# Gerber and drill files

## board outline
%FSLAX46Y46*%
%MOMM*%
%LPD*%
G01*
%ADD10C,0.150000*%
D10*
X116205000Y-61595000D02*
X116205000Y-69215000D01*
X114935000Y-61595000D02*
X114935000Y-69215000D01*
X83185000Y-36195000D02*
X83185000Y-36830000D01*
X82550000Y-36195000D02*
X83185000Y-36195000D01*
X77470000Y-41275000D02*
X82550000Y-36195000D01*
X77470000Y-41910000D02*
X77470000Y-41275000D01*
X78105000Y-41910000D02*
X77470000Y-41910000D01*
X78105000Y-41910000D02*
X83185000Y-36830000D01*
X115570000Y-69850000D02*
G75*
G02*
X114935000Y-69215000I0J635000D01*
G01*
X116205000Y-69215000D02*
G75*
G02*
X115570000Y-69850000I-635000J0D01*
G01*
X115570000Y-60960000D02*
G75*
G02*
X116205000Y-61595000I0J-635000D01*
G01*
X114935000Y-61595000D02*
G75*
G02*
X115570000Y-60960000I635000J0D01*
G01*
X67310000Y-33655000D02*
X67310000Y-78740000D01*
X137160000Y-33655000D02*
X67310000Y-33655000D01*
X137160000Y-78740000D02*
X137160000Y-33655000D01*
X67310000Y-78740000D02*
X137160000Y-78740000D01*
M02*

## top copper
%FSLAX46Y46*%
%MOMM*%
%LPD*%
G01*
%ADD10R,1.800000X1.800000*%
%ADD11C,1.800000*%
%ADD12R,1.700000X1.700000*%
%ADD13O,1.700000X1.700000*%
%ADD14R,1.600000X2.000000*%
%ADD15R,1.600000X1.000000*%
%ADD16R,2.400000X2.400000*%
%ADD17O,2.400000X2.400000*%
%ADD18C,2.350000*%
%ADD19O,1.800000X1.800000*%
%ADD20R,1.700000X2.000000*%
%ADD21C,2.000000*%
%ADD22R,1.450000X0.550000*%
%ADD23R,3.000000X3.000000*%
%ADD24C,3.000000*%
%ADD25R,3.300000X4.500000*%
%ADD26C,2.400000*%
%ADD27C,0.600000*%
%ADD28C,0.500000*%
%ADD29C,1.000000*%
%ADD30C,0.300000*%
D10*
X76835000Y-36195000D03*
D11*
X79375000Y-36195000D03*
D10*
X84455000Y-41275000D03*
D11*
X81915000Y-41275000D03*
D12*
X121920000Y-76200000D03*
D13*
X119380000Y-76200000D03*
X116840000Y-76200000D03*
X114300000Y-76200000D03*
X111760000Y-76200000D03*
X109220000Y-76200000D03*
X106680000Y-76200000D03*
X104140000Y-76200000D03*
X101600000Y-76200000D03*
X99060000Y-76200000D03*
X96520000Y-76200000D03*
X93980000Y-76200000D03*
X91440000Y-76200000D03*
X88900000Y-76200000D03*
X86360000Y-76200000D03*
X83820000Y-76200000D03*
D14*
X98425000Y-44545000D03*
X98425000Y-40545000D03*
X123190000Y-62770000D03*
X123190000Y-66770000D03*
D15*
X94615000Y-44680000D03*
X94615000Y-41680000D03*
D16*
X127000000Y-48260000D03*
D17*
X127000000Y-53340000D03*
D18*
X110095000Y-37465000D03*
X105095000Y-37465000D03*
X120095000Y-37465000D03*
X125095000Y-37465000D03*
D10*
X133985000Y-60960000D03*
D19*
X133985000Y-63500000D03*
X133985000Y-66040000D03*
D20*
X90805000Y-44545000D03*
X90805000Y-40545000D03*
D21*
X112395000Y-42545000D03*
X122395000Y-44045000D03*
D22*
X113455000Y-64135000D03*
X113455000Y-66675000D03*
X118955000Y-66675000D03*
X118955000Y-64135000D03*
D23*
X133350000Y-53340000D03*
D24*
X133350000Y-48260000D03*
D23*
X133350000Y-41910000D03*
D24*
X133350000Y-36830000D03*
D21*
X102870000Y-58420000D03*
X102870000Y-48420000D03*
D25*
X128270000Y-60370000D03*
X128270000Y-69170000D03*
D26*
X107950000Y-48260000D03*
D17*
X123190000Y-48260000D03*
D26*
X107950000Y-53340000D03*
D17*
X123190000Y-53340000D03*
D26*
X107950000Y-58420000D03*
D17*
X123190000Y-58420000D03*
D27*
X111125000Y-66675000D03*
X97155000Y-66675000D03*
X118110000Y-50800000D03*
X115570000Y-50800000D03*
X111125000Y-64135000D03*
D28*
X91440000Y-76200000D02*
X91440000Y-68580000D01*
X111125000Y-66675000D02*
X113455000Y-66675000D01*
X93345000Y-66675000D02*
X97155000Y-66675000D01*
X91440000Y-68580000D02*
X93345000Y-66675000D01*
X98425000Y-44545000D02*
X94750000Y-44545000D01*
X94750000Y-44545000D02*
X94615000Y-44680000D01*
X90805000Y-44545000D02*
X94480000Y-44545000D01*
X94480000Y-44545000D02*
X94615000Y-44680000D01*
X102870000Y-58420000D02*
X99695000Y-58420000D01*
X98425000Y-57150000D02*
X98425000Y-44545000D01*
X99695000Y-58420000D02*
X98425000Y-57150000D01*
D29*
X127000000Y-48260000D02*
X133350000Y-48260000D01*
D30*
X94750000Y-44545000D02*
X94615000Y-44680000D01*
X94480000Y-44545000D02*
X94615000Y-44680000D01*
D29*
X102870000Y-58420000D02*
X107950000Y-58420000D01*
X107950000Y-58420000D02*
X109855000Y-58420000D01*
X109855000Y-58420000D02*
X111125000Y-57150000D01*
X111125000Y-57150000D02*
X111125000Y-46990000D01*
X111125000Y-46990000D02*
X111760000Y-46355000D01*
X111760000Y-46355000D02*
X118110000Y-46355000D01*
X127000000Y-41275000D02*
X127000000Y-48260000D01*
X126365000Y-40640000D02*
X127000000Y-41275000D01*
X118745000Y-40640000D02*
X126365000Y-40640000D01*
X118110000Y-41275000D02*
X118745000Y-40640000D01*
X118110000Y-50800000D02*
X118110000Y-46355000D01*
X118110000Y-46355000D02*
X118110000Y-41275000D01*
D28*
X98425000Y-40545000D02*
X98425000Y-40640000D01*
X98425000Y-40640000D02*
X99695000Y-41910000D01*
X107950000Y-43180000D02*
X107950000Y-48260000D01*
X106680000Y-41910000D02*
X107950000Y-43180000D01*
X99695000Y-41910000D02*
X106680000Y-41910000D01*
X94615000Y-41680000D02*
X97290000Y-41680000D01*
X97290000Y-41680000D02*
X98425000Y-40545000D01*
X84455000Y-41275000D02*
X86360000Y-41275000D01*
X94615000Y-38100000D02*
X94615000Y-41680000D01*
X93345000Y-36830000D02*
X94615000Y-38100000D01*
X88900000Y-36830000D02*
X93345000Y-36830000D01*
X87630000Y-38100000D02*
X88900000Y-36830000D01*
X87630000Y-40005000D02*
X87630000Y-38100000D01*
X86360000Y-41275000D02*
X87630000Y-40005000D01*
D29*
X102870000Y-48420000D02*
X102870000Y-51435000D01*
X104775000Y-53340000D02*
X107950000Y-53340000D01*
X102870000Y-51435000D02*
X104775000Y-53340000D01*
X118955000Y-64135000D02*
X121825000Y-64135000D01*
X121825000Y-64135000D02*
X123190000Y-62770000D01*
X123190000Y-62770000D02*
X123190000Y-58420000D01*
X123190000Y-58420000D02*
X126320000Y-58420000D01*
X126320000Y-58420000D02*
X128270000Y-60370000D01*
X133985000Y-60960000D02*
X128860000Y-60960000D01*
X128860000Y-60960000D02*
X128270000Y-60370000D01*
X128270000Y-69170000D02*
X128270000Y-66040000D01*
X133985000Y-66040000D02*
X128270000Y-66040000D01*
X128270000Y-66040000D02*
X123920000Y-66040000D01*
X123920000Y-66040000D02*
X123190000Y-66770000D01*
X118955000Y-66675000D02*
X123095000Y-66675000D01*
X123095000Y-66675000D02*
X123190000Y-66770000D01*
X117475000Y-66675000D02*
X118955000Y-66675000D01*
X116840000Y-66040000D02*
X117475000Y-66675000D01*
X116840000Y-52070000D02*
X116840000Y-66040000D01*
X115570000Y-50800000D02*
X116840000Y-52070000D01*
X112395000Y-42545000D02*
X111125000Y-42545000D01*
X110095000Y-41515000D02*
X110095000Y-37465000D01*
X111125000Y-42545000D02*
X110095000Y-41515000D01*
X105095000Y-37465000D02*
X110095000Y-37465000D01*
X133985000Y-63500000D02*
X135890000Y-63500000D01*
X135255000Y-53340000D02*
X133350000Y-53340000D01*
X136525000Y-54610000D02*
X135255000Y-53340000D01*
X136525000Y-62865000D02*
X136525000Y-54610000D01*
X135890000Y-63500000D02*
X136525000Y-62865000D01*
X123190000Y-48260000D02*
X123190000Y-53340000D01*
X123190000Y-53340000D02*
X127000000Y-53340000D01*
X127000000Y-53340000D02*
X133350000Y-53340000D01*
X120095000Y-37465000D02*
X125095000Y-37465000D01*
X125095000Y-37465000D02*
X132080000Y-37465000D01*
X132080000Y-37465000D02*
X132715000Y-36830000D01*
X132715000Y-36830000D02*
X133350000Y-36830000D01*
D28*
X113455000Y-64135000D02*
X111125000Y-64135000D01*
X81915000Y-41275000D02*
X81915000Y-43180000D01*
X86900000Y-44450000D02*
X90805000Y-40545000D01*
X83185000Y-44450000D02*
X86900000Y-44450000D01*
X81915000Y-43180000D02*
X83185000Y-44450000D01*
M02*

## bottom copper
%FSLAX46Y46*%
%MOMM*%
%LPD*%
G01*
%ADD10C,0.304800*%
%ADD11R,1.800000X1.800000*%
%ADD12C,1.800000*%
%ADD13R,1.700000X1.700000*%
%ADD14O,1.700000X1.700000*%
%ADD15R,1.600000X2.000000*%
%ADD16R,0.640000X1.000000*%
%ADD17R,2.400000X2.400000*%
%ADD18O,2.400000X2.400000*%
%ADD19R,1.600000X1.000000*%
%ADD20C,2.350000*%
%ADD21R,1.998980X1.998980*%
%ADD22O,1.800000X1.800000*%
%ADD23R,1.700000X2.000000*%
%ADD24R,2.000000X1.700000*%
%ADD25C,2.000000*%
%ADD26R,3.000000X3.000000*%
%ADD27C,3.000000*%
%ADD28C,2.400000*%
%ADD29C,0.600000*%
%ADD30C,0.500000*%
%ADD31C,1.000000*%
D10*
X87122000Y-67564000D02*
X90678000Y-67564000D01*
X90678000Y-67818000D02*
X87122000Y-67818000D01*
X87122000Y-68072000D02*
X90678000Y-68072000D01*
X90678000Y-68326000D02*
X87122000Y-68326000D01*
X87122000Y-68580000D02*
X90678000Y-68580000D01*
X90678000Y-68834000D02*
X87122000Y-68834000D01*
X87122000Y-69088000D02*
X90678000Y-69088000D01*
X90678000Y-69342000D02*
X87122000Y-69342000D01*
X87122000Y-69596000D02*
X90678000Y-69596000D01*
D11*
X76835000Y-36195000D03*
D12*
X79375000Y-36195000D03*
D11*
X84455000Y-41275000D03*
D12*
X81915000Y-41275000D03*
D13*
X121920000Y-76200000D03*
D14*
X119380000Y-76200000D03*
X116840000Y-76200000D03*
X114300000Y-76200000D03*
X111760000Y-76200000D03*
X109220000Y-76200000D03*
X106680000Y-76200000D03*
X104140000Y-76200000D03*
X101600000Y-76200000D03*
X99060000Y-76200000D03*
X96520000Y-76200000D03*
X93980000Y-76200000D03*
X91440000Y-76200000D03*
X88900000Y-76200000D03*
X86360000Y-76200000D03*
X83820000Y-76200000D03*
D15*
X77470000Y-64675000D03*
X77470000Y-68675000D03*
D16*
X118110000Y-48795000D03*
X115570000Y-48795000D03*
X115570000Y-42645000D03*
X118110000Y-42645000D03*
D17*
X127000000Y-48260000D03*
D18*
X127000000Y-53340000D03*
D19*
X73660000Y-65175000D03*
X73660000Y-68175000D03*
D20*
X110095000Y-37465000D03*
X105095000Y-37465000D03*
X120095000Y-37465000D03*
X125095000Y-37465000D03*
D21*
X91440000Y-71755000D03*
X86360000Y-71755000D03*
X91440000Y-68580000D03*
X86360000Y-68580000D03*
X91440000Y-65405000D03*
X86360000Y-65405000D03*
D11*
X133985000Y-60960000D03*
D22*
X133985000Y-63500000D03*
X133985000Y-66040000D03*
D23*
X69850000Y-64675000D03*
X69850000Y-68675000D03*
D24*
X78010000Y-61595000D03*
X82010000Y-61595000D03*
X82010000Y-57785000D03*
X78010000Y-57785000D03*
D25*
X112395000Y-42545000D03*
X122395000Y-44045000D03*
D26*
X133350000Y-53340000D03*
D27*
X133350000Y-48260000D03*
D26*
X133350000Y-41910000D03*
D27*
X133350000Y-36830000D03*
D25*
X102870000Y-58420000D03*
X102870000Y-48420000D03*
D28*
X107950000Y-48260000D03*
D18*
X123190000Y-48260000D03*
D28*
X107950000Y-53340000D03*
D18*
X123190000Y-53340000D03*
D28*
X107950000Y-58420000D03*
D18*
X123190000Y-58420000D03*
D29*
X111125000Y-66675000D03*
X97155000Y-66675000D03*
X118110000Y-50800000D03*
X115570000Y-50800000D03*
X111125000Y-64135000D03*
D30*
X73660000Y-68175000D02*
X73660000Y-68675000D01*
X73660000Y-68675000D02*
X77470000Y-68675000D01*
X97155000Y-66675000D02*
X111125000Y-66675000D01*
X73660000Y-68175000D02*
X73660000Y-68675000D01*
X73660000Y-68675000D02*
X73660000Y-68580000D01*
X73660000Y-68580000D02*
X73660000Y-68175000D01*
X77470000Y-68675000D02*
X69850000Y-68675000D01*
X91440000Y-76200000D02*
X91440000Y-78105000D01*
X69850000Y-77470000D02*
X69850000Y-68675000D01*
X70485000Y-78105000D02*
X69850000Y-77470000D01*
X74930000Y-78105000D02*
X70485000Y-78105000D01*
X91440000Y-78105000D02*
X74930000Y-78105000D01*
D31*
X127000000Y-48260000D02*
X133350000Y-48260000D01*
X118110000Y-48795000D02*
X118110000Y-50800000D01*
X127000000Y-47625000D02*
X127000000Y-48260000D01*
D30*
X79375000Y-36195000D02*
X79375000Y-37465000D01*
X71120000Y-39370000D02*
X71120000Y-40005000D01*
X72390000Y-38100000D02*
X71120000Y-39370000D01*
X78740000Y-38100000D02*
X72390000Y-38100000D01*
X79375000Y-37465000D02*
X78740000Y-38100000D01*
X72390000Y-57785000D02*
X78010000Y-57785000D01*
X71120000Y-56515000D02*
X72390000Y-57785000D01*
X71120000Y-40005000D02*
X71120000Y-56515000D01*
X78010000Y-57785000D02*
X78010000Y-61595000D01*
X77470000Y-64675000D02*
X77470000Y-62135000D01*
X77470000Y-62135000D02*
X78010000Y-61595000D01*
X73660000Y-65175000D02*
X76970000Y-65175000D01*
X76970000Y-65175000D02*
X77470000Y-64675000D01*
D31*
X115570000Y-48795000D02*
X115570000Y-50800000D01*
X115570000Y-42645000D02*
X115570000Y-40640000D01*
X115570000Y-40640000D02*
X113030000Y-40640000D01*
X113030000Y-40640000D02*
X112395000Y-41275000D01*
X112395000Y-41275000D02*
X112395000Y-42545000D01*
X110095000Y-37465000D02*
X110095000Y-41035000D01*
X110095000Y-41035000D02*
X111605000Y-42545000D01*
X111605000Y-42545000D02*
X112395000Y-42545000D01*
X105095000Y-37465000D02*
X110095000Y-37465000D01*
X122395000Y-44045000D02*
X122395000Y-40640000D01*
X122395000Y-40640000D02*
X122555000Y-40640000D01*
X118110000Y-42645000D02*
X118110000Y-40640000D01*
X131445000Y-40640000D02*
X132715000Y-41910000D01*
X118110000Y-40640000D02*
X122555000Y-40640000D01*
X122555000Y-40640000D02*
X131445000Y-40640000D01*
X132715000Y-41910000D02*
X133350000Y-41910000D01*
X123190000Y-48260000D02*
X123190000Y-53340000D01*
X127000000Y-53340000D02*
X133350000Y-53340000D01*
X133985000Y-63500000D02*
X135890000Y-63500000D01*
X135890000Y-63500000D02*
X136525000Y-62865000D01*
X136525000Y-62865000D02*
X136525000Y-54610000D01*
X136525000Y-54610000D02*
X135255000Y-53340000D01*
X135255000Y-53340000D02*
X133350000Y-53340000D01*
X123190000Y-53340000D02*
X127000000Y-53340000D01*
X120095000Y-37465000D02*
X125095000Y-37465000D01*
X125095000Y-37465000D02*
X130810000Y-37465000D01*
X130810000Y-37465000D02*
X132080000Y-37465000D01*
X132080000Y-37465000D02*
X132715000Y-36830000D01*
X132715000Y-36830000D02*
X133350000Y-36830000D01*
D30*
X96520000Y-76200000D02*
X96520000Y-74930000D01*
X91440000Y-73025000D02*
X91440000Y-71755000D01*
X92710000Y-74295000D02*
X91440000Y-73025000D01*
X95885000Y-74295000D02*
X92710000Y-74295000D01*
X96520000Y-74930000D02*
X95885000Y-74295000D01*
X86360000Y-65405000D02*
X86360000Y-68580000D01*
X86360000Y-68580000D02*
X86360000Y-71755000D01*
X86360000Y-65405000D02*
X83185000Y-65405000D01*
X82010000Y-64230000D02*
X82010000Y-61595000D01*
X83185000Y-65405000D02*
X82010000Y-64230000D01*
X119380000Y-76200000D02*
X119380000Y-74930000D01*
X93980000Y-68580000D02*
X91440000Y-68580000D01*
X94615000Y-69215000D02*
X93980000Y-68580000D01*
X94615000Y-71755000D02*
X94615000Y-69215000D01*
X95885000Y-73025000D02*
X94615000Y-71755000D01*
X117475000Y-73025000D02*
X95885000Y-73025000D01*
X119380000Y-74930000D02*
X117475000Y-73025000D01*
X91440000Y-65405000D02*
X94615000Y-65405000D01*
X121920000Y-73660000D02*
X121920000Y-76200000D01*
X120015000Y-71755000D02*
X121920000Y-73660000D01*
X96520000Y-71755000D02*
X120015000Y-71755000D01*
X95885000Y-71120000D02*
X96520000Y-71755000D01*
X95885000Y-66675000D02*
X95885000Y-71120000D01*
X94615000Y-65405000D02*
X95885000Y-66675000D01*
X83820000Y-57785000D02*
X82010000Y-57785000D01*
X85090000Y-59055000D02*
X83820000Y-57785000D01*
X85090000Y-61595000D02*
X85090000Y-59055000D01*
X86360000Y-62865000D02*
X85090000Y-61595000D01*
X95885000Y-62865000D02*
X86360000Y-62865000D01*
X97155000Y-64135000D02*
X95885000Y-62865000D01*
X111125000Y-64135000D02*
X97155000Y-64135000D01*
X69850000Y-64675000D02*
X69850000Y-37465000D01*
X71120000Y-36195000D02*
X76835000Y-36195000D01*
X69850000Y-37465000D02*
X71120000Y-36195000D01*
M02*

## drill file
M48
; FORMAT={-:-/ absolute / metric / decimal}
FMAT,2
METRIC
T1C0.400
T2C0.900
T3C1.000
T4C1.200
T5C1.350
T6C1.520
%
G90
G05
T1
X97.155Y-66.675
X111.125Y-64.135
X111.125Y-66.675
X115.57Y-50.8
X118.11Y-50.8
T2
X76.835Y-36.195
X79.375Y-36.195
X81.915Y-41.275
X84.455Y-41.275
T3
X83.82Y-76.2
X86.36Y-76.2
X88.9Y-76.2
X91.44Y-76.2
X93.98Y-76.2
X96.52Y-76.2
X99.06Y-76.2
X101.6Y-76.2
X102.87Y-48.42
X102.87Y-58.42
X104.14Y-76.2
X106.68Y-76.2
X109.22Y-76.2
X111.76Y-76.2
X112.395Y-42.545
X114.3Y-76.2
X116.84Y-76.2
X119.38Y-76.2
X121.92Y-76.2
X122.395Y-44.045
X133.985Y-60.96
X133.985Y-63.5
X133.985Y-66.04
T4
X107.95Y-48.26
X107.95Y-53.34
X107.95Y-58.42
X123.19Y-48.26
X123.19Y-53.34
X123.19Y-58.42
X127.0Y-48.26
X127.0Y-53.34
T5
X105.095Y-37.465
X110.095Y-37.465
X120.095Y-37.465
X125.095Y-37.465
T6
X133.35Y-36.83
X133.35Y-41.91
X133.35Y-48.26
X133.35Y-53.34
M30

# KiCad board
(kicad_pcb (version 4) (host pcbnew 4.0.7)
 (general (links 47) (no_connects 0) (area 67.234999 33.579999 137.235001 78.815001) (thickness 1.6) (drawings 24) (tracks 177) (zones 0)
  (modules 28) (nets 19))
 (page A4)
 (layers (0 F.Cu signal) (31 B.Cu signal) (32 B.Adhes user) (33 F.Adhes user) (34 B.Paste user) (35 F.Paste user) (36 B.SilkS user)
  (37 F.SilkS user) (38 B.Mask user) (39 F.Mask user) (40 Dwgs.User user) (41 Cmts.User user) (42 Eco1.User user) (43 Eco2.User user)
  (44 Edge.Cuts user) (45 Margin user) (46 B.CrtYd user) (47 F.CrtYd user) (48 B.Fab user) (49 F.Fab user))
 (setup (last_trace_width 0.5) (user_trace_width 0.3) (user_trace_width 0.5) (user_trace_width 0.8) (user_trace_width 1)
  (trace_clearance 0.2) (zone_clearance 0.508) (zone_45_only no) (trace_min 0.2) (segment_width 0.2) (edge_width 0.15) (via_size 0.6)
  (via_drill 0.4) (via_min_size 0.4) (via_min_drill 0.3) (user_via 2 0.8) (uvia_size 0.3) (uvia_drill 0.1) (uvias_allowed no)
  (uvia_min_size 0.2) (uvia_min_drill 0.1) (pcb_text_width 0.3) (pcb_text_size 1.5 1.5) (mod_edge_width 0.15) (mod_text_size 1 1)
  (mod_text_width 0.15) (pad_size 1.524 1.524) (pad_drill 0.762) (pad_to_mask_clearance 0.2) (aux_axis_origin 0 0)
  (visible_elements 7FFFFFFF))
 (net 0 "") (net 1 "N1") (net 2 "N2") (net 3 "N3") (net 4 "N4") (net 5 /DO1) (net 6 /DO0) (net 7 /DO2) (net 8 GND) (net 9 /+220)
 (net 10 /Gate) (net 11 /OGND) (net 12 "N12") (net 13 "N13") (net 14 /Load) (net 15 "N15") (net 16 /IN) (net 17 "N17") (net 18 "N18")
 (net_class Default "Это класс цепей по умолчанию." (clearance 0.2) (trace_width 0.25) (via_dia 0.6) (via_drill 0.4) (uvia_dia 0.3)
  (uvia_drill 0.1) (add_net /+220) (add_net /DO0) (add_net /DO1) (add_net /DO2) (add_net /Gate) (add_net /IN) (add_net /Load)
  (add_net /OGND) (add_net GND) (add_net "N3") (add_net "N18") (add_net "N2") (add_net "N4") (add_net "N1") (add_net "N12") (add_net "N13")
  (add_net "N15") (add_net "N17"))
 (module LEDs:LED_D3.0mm (layer F.Cu) (at 76.835 36.195)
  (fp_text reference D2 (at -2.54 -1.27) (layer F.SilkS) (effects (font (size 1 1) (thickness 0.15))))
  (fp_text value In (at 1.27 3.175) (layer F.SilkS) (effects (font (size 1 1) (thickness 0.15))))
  (pad 1 thru_hole rect (at 0 0) (size 1.8 1.8) (drill 0.9) (layers *.Cu *.Mask) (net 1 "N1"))
  (pad 2 thru_hole circle (at 2.54 0) (size 1.8 1.8) (drill 0.9) (layers *.Cu *.Mask) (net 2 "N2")))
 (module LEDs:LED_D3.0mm (layer F.Cu) (at 84.455 41.275 180)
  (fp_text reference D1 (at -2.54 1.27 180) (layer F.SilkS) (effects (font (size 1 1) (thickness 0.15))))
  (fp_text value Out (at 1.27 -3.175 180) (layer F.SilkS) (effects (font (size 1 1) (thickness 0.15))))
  (pad 1 thru_hole rect (at 0 0 180) (size 1.8 1.8) (drill 0.9) (layers *.Cu *.Mask) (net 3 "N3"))
  (pad 2 thru_hole circle (at 2.54 0 180) (size 1.8 1.8) (drill 0.9) (layers *.Cu *.Mask) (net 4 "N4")))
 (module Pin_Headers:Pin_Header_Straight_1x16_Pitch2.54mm (layer F.Cu) (at 121.92 76.2 270)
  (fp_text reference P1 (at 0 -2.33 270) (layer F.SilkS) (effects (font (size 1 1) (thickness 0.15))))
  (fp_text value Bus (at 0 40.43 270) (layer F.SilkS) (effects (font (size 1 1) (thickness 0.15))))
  (pad 1 thru_hole rect (at 0 0 270) (size 1.7 1.7) (drill 1) (layers *.Cu *.Mask) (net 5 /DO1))
  (pad 2 thru_hole oval (at 0 2.54 270) (size 1.7 1.7) (drill 1) (layers *.Cu *.Mask) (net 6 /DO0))
  (pad 3 thru_hole oval (at 0 5.08 270) (size 1.7 1.7) (drill 1) (layers *.Cu *.Mask))
  (pad 4 thru_hole oval (at 0 7.62 270) (size 1.7 1.7) (drill 1) (layers *.Cu *.Mask))
  (pad 5 thru_hole oval (at 0 10.16 270) (size 1.7 1.7) (drill 1) (layers *.Cu *.Mask))
  (pad 6 thru_hole oval (at 0 12.7 270) (size 1.7 1.7) (drill 1) (layers *.Cu *.Mask))
  (pad 7 thru_hole oval (at 0 15.24 270) (size 1.7 1.7) (drill 1) (layers *.Cu *.Mask))
  (pad 8 thru_hole oval (at 0 17.78 270) (size 1.7 1.7) (drill 1) (layers *.Cu *.Mask))
  (pad 9 thru_hole oval (at 0 20.32 270) (size 1.7 1.7) (drill 1) (layers *.Cu *.Mask))
  (pad 10 thru_hole oval (at 0 22.86 270) (size 1.7 1.7) (drill 1) (layers *.Cu *.Mask))
  (pad 11 thru_hole oval (at 0 25.4 270) (size 1.7 1.7) (drill 1) (layers *.Cu *.Mask) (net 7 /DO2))
  (pad 12 thru_hole oval (at 0 27.94 270) (size 1.7 1.7) (drill 1) (layers *.Cu *.Mask))
  (pad 13 thru_hole oval (at 0 30.48 270) (size 1.7 1.7) (drill 1) (layers *.Cu *.Mask) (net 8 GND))
  (pad 14 thru_hole oval (at 0 33.02 270) (size 1.7 1.7) (drill 1) (layers *.Cu *.Mask))
  (pad 15 thru_hole oval (at 0 35.56 270) (size 1.7 1.7) (drill 1) (layers *.Cu *.Mask))
  (pad 16 thru_hole oval (at 0 38.1 270) (size 1.7 1.7) (drill 1) (layers *.Cu *.Mask)))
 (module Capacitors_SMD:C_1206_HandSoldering (layer F.Cu) (at 98.425 42.545 90)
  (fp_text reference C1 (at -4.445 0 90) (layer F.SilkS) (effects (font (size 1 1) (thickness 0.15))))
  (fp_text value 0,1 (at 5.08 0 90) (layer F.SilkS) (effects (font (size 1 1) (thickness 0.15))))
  (pad 1 smd rect (at -2 0 90) (size 2 1.6) (layers F.Cu F.Paste F.Mask) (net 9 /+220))
  (pad 2 smd rect (at 2 0 90) (size 2 1.6) (layers F.Cu F.Paste F.Mask) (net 3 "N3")))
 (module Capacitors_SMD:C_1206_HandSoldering (layer B.Cu) (at 77.47 66.675 270)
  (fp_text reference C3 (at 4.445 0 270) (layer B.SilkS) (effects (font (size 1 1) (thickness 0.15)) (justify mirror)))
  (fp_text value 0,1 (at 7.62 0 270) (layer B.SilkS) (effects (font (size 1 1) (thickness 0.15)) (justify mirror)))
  (pad 1 smd rect (at -2 0 270) (size 2 1.6) (layers B.Cu B.Paste B.Mask) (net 2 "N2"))
  (pad 2 smd rect (at 2 0 270) (size 2 1.6) (layers B.Cu B.Paste B.Mask) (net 8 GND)))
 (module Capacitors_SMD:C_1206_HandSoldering (layer F.Cu) (at 123.19 64.77 270)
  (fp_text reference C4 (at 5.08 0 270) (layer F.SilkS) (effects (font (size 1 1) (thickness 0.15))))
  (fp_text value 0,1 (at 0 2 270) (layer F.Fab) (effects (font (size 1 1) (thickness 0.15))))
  (pad 1 smd rect (at -2 0 270) (size 2 1.6) (layers F.Cu F.Paste F.Mask) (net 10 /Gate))
  (pad 2 smd rect (at 2 0 270) (size 2 1.6) (layers F.Cu F.Paste F.Mask) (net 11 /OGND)))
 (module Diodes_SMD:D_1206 (layer F.Cu) (at 94.615 43.18 90)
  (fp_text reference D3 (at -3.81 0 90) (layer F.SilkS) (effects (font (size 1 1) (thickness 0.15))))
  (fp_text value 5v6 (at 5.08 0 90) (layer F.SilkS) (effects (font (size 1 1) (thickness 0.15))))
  (pad 1 smd rect (at -1.5 0 90) (size 1 1.6) (layers F.Cu F.Paste F.Mask) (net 9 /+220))
  (pad 2 smd rect (at 1.5 0 90) (size 1 1.6) (layers F.Cu F.Paste F.Mask) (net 3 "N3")))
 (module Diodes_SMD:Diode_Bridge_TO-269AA (layer B.Cu) (at 116.84 45.72 90)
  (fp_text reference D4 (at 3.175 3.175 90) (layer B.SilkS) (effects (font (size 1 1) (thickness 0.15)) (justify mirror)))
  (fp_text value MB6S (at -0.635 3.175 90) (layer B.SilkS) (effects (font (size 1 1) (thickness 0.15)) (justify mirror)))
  (pad 1 smd rect (at -3.075 1.27 90) (size 1 0.64) (layers B.Cu B.Paste B.Mask) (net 9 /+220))
  (pad 2 smd rect (at -3.075 -1.27 90) (size 1 0.64) (layers B.Cu B.Paste B.Mask) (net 11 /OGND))
  (pad 3 smd rect (at 3.075 -1.27 90) (size 1 0.64) (layers B.Cu B.Paste B.Mask) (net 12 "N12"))
  (pad 4 smd rect (at 3.075 1.27 90) (size 1 0.64) (layers B.Cu B.Paste B.Mask) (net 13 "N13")))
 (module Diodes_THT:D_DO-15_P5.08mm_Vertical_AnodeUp (layer F.Cu) (at 127 48.26 270)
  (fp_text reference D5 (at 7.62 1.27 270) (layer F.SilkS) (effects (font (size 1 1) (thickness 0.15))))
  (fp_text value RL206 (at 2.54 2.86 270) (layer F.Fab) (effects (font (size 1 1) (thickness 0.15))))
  (pad 1 thru_hole rect (at 0 0 270) (size 2.4 2.4) (drill 1.2) (layers *.Cu *.Mask) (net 9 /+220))
  (pad 2 thru_hole oval (at 5.08 0 270) (size 2.4 2.4) (drill 1.2) (layers *.Cu *.Mask) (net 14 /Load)))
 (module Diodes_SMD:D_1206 (layer B.Cu) (at 73.66 66.675 270)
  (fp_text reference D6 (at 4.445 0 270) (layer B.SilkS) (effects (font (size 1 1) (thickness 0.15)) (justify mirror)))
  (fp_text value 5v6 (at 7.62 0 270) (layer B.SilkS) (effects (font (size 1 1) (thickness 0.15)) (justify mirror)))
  (pad 1 smd rect (at -1.5 0 270) (size 1 1.6) (layers B.Cu B.Paste B.Mask) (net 2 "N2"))
  (pad 2 smd rect (at 1.5 0 270) (size 1 1.6) (layers B.Cu B.Paste B.Mask) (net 8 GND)))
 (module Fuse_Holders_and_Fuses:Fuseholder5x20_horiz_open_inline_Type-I (layer F.Cu) (at 125.095 37.465 180)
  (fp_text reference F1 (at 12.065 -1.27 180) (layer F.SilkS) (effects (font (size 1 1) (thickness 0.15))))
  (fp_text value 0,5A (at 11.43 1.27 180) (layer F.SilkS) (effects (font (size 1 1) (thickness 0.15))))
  (pad 2 thru_hole circle (at 15 0 180) (size 2.35 2.35) (drill 1.35) (layers *.Cu *.Mask) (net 12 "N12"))
  (pad 2 thru_hole circle (at 20 0 180) (size 2.35 2.35) (drill 1.35) (layers *.Cu *.Mask) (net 12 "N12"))
  (pad 1 thru_hole circle (at 5 0 180) (size 2.35 2.35) (drill 1.35) (layers *.Cu *.Mask) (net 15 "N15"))
  (pad 1 thru_hole circle (at 0 0 180) (size 2.35 2.35) (drill 1.35) (layers *.Cu *.Mask) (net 15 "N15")))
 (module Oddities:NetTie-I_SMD (layer B.Cu) (at 88.9 71.755 180)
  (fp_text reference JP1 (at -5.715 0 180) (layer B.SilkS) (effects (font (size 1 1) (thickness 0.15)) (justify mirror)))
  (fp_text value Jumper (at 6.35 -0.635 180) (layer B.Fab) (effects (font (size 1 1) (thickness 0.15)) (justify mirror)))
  (pad 1 smd rect (at -2.54 0 180) (size 1.99898 1.99898) (layers B.Cu B.Paste B.Mask) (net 7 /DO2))
  (pad 2 smd rect (at 2.54 0 180) (size 1.99898 1.99898) (layers B.Cu B.Paste B.Mask) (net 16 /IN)))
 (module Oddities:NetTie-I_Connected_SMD (layer B.Cu) (at 88.9 68.58 180)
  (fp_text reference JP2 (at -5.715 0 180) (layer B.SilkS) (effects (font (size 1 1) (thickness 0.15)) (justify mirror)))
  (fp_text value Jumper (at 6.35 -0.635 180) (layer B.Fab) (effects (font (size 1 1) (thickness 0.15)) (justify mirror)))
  (fp_line (start 1.778 1.016) (end -1.778 1.016) (layer B.Cu) (width 0.3048))
  (fp_line (start -1.778 0.762) (end 1.778 0.762) (layer B.Cu) (width 0.3048))
  (fp_line (start 1.778 0.508) (end -1.778 0.508) (layer B.Cu) (width 0.3048))
  (fp_line (start -1.778 0.254) (end 1.778 0.254) (layer B.Cu) (width 0.3048))
  (fp_line (start 1.778 0) (end -1.778 0) (layer B.Cu) (width 0.3048))
  (fp_line (start -1.778 -0.254) (end 1.778 -0.254) (layer B.Cu) (width 0.3048))
  (fp_line (start 1.778 -0.508) (end -1.778 -0.508) (layer B.Cu) (width 0.3048))
  (fp_line (start -1.778 -0.762) (end 1.778 -0.762) (layer B.Cu) (width 0.3048))
  (fp_line (start 1.778 -1.016) (end -1.778 -1.016) (layer B.Cu) (width 0.3048))
  (pad 1 smd rect (at -2.54 0 180) (size 1.99898 1.99898) (layers B.Cu B.Paste B.Mask) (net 6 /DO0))
  (pad 2 smd rect (at 2.54 0 180) (size 1.99898 1.99898) (layers B.Cu B.Paste B.Mask) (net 16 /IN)))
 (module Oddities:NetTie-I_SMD (layer B.Cu) (at 88.9 65.405 180)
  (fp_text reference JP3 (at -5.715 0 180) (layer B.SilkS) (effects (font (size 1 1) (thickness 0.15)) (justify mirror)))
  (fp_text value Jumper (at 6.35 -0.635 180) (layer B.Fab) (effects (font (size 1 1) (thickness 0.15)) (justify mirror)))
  (pad 1 smd rect (at -2.54 0 180) (size 1.99898 1.99898) (layers B.Cu B.Paste B.Mask) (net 5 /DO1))
  (pad 2 smd rect (at 2.54 0 180) (size 1.99898 1.99898) (layers B.Cu B.Paste B.Mask) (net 16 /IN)))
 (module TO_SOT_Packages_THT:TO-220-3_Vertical (layer F.Cu) (at 133.985 60.96 270)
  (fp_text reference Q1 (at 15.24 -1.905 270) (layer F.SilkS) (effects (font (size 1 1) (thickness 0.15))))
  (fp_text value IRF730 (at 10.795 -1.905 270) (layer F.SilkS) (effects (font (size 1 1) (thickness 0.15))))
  (pad 1 thru_hole rect (at 0 0 270) (size 1.8 1.8) (drill 1) (layers *.Cu *.Mask) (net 10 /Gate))
  (pad 2 thru_hole oval (at 2.54 0 270) (size 1.8 1.8) (drill 1) (layers *.Cu *.Mask) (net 14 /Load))
  (pad 3 thru_hole oval (at 5.08 0 270) (size 1.8 1.8) (drill 1) (layers *.Cu *.Mask) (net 11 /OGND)))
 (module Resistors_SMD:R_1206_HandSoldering (layer F.Cu) (at 90.805 42.545 90)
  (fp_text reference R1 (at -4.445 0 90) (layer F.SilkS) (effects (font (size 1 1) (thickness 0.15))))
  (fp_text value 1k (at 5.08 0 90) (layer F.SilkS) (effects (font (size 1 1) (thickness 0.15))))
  (pad 1 smd rect (at -2 0 90) (size 2 1.7) (layers F.Cu F.Paste F.Mask) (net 9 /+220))
  (pad 2 smd rect (at 2 0 90) (size 2 1.7) (layers F.Cu F.Paste F.Mask) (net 4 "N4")))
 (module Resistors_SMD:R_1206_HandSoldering (layer B.Cu) (at 69.85 66.675 270)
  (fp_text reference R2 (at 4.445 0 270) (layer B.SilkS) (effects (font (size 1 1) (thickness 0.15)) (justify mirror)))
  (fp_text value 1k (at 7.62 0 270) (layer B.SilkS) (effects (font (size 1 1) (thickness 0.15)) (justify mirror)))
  (pad 1 smd rect (at -2 0 270) (size 2 1.7) (layers B.Cu B.Paste B.Mask) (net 1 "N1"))
  (pad 2 smd rect (at 2 0 270) (size 2 1.7) (layers B.Cu B.Paste B.Mask) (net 8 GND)))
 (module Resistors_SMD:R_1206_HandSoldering (layer B.Cu) (at 80.01 61.595)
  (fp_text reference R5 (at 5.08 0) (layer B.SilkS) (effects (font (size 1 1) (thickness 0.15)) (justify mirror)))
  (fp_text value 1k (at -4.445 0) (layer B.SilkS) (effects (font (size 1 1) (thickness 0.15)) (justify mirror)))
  (pad 1 smd rect (at -2 0) (size 2 1.7) (layers B.Cu B.Paste B.Mask) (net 2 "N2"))
  (pad 2 smd rect (at 2 0) (size 2 1.7) (layers B.Cu B.Paste B.Mask) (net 16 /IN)))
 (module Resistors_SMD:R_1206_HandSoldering (layer B.Cu) (at 80.01 57.785 180)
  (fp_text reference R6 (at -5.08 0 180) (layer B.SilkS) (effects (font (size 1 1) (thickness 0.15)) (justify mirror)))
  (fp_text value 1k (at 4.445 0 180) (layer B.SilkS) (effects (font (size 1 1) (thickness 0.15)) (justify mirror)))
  (pad 1 smd rect (at -2 0 180) (size 2 1.7) (layers B.Cu B.Paste B.Mask) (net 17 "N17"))
  (pad 2 smd rect (at 2 0 180) (size 2 1.7) (layers B.Cu B.Paste B.Mask) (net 2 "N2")))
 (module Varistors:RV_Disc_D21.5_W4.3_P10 (layer F.Cu) (at 112.395 42.545)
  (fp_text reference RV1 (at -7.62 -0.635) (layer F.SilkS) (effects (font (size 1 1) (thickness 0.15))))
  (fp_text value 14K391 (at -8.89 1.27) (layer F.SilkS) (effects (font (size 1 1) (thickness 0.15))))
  (pad 1 thru_hole circle (at 0 0) (size 2 2) (drill 1) (layers *.Cu *.Mask) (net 12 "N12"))
  (pad 2 thru_hole circle (at 10 1.5) (size 2 2) (drill 1) (layers *.Cu *.Mask) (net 13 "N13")))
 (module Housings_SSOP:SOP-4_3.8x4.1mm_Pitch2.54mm (layer F.Cu) (at 116.205 65.405)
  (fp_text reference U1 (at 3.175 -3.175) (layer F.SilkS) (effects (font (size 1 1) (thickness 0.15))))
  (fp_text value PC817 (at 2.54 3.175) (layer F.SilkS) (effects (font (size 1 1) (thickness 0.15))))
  (pad 1 smd rect (at -2.75 -1.27) (size 1.45 0.55) (layers F.Cu F.Paste F.Mask) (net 17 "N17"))
  (pad 2 smd rect (at -2.75 1.27) (size 1.45 0.55) (layers F.Cu F.Paste F.Mask) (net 8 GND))
  (pad 3 smd rect (at 2.75 1.27) (size 1.45 0.55) (layers F.Cu F.Paste F.Mask) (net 11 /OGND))
  (pad 4 smd rect (at 2.75 -1.27) (size 1.45 0.55) (layers F.Cu F.Paste F.Mask) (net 10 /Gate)))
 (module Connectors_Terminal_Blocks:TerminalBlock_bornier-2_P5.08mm (layer F.Cu) (at 133.35 53.34 90)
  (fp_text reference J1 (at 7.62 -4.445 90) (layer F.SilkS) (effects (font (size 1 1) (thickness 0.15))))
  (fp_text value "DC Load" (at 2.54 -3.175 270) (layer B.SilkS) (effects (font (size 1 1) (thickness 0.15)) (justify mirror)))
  (pad 1 thru_hole rect (at 0 0 90) (size 3 3) (drill 1.52) (layers *.Cu *.Mask) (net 14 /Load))
  (pad 2 thru_hole circle (at 5.08 0 90) (size 3 3) (drill 1.52) (layers *.Cu *.Mask) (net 9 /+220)))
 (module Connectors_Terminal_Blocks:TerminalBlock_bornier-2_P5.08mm (layer F.Cu) (at 133.35 41.91 90)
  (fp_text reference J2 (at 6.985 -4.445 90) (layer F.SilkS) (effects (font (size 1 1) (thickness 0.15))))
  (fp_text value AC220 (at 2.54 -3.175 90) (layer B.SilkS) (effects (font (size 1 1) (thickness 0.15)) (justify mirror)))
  (pad 1 thru_hole rect (at 0 0 90) (size 3 3) (drill 1.52) (layers *.Cu *.Mask) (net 13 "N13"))
  (pad 2 thru_hole circle (at 5.08 0 90) (size 3 3) (drill 1.52) (layers *.Cu *.Mask) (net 15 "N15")))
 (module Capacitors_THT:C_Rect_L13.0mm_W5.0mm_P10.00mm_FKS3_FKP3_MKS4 (layer F.Cu) (at 102.87 58.42 90)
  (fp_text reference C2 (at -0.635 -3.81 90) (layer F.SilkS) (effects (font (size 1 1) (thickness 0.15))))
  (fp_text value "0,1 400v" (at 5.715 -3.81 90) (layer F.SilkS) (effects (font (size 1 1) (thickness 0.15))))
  (pad 1 thru_hole circle (at 0 0 90) (size 2 2) (drill 1) (layers *.Cu *.Mask) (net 9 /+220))
  (pad 2 thru_hole circle (at 10 0 90) (size 2 2) (drill 1) (layers *.Cu *.Mask) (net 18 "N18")))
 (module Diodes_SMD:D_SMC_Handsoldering (layer F.Cu) (at 128.27 64.77 270)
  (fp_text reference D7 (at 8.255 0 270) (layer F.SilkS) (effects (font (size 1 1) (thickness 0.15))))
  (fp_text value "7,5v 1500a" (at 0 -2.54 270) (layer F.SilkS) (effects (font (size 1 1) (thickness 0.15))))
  (pad 1 smd rect (at -4.4 0) (size 3.3 4.5) (layers F.Cu F.Paste F.Mask) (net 10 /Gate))
  (pad 2 smd rect (at 4.4 0) (size 3.3 4.5) (layers F.Cu F.Paste F.Mask) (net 11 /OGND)))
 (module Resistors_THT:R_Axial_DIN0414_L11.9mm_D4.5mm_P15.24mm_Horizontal (layer F.Cu) (at 107.95 48.26)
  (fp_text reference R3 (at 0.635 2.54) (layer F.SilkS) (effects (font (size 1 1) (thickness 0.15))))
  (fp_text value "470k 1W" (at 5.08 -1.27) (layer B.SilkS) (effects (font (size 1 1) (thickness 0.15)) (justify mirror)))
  (pad 1 thru_hole circle (at 0 0) (size 2.4 2.4) (drill 1.2) (layers *.Cu *.Mask) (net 3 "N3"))
  (pad 2 thru_hole oval (at 15.24 0) (size 2.4 2.4) (drill 1.2) (layers *.Cu *.Mask) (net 14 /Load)))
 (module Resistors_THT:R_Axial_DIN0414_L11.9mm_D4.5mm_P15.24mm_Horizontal (layer F.Cu) (at 107.95 53.34)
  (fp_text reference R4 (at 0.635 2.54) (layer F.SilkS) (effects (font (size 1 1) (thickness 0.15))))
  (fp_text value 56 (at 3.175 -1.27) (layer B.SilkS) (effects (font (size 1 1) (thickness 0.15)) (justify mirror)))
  (pad 1 thru_hole circle (at 0 0) (size 2.4 2.4) (drill 1.2) (layers *.Cu *.Mask) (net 18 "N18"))
  (pad 2 thru_hole oval (at 15.24 0) (size 2.4 2.4) (drill 1.2) (layers *.Cu *.Mask) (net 14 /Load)))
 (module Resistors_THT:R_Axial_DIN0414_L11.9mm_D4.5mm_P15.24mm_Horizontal (layer F.Cu) (at 107.95 58.42)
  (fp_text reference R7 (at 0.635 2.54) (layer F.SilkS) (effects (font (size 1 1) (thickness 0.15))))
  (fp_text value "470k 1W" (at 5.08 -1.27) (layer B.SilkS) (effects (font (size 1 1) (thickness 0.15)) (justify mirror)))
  (pad 1 thru_hole circle (at 0 0) (size 2.4 2.4) (drill 1.2) (layers *.Cu *.Mask) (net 9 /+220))
  (pad 2 thru_hole oval (at 15.24 0) (size 2.4 2.4) (drill 1.2) (layers *.Cu *.Mask) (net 10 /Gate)))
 (gr_line (start 116.205 61.595) (end 116.205 69.215) (angle 90) (layer Edge.Cuts) (width 0.15))
 (gr_line (start 114.935 61.595) (end 114.935 69.215) (angle 90) (layer Edge.Cuts) (width 0.15))
 (gr_line (start 83.185 36.195) (end 83.185 36.83) (angle 90) (layer Edge.Cuts) (width 0.15))
 (gr_line (start 82.55 36.195) (end 83.185 36.195) (angle 90) (layer Edge.Cuts) (width 0.15))
 (gr_line (start 77.47 41.275) (end 82.55 36.195) (angle 90) (layer Edge.Cuts) (width 0.15))
 (gr_line (start 77.47 41.91) (end 77.47 41.275) (angle 90) (layer Edge.Cuts) (width 0.15))
 (gr_line (start 78.105 41.91) (end 77.47 41.91) (angle 90) (layer Edge.Cuts) (width 0.15))
 (gr_line (start 78.105 41.91) (end 83.185 36.83) (angle 90) (layer Edge.Cuts) (width 0.15))
 (gr_arc (start 115.57 69.215) (end 115.57 69.85) (angle 90) (layer Edge.Cuts) (width 0.15))
 (gr_arc (start 115.57 69.215) (end 116.205 69.215) (angle 90) (layer Edge.Cuts) (width 0.15))
 (gr_arc (start 115.57 61.595) (end 115.57 60.96) (angle 90) (layer Edge.Cuts) (width 0.15))
 (gr_arc (start 115.57 61.595) (end 114.935 61.595) (angle 90) (layer Edge.Cuts) (width 0.15))
 (gr_line (start 67.31 33.655) (end 67.31 78.74) (angle 90) (layer Edge.Cuts) (width 0.15))
 (gr_line (start 137.16 33.655) (end 67.31 33.655) (angle 90) (layer Edge.Cuts) (width 0.15))
 (gr_line (start 137.16 78.74) (end 137.16 33.655) (angle 90) (layer Edge.Cuts) (width 0.15))
 (gr_line (start 67.31 78.74) (end 137.16 78.74) (angle 90) (layer Edge.Cuts) (width 0.15))
 (segment (start 73.66 68.175) (end 73.66 68.675) (width 0.5) (layer B.Cu) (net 8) (status C00000))
 (segment (start 73.66 68.675) (end 77.47 68.675) (width 0.5) (layer B.Cu) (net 8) (status C00000))
 (segment (start 91.44 76.2) (end 91.44 68.58) (width 0.5) (layer F.Cu) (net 8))
 (via (at 111.125 66.675) (size 0.6) (drill 0.4) (layers F.Cu B.Cu) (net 8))
 (segment (start 111.125 66.675) (end 113.455 66.675) (width 0.5) (layer F.Cu) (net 8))
 (segment (start 97.155 66.675) (end 111.125 66.675) (width 0.5) (layer B.Cu) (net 8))
 (via (at 97.155 66.675) (size 0.6) (drill 0.4) (layers F.Cu B.Cu) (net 8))
 (segment (start 93.345 66.675) (end 97.155 66.675) (width 0.5) (layer F.Cu) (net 8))
 (segment (start 91.44 68.58) (end 93.345 66.675) (width 0.5) (layer F.Cu) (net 8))
 (segment (start 73.66 68.175) (end 73.66 68.675) (width 0.5) (layer B.Cu) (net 8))
 (segment (start 73.66 68.675) (end 73.66 68.58) (width 0.5) (layer B.Cu) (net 8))
 (segment (start 73.66 68.58) (end 73.66 68.175) (width 0.5) (layer B.Cu) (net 8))
 (segment (start 77.47 68.675) (end 69.85 68.675) (width 0.5) (layer B.Cu) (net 8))
 (segment (start 91.44 76.2) (end 91.44 78.105) (width 0.5) (layer B.Cu) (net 8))
 (segment (start 69.85 77.47) (end 69.85 68.675) (width 0.5) (layer B.Cu) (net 8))
 (segment (start 70.485 78.105) (end 69.85 77.47) (width 0.5) (layer B.Cu) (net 8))
 (segment (start 74.93 78.105) (end 70.485 78.105) (width 0.5) (layer B.Cu) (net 8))
 (segment (start 91.44 78.105) (end 74.93 78.105) (width 0.5) (layer B.Cu) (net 8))
 (segment (start 98.425 44.545) (end 94.75 44.545) (width 0.5) (layer F.Cu) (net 9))
 (segment (start 94.75 44.545) (end 94.615 44.68) (width 0.5) (layer F.Cu) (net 9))
 (segment (start 90.805 44.545) (end 94.48 44.545) (width 0.5) (layer F.Cu) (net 9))
 (segment (start 94.48 44.545) (end 94.615 44.68) (width 0.5) (layer F.Cu) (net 9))
 (segment (start 102.87 58.42) (end 99.695 58.42) (width 0.5) (layer F.Cu) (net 9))
 (segment (start 98.425 57.15) (end 98.425 44.545) (width 0.5) (layer F.Cu) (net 9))
 (segment (start 99.695 58.42) (end 98.425 57.15) (width 0.5) (layer F.Cu) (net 9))
 (segment (start 127 48.26) (end 133.35 48.26) (width 1) (layer B.Cu) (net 9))
 (segment (start 127 48.26) (end 133.35 48.26) (width 1) (layer F.Cu) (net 9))
 (segment (start 94.75 44.545) (end 94.615 44.68) (width 0.3) (layer F.Cu) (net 9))
 (segment (start 94.48 44.545) (end 94.615 44.68) (width 0.3) (layer F.Cu) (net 9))
 (segment (start 102.87 58.42) (end 107.95 58.42) (width 1) (layer F.Cu) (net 9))
 (segment (start 107.95 58.42) (end 109.855 58.42) (width 1) (layer F.Cu) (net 9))
 (segment (start 109.855 58.42) (end 111.125 57.15) (width 1) (layer F.Cu) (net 9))
 (segment (start 111.125 57.15) (end 111.125 46.99) (width 1) (layer F.Cu) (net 9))
 (segment (start 111.125 46.99) (end 111.76 46.355) (width 1) (layer F.Cu) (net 9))
 (segment (start 111.76 46.355) (end 118.11 46.355) (width 1) (layer F.Cu) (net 9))
 (segment (start 118.11 48.795) (end 118.11 50.8) (width 1) (layer B.Cu) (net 9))
 (segment (start 127 41.275) (end 127 48.26) (width 1) (layer F.Cu) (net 9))
 (segment (start 126.365 40.64) (end 127 41.275) (width 1) (layer F.Cu) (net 9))
 (segment (start 118.745 40.64) (end 126.365 40.64) (width 1) (layer F.Cu) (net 9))
 (segment (start 118.11 41.275) (end 118.745 40.64) (width 1) (layer F.Cu) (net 9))
 (segment (start 118.11 50.8) (end 118.11 46.355) (width 1) (layer F.Cu) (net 9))
 (segment (start 118.11 46.355) (end 118.11 41.275) (width 1) (layer F.Cu) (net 9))
 (via (at 118.11 50.8) (size 0.6) (drill 0.4) (layers F.Cu B.Cu) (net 9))
 (segment (start 127 47.625) (end 127 48.26) (width 1) (layer B.Cu) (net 9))
 (segment (start 98.425 40.545) (end 98.425 40.64) (width 0.5) (layer F.Cu) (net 3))
 (segment (start 98.425 40.64) (end 99.695 41.91) (width 0.5) (layer F.Cu) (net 3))
 (segment (start 107.95 43.18) (end 107.95 48.26) (width 0.5) (layer F.Cu) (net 3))
 (segment (start 106.68 41.91) (end 107.95 43.18) (width 0.5) (layer F.Cu) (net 3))
 (segment (start 99.695 41.91) (end 106.68 41.91) (width 0.5) (layer F.Cu) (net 3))
 (segment (start 94.615 41.68) (end 97.29 41.68) (width 0.5) (layer F.Cu) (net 3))
 (segment (start 97.29 41.68) (end 98.425 40.545) (width 0.5) (layer F.Cu) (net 3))
 (segment (start 84.455 41.275) (end 86.36 41.275) (width 0.5) (layer F.Cu) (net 3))
 (segment (start 94.615 38.1) (end 94.615 41.68) (width 0.5) (layer F.Cu) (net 3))
 (segment (start 93.345 36.83) (end 94.615 38.1) (width 0.5) (layer F.Cu) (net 3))
 (segment (start 88.9 36.83) (end 93.345 36.83) (width 0.5) (layer F.Cu) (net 3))
 (segment (start 87.63 38.1) (end 88.9 36.83) (width 0.5) (layer F.Cu) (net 3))
 (segment (start 87.63 40.005) (end 87.63 38.1) (width 0.5) (layer F.Cu) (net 3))
 (segment (start 86.36 41.275) (end 87.63 40.005) (width 0.5) (layer F.Cu) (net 3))
 (segment (start 102.87 48.42) (end 102.87 51.435) (width 1) (layer F.Cu) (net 18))
 (segment (start 104.775 53.34) (end 107.95 53.34) (width 1) (layer F.Cu) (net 18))
 (segment (start 102.87 51.435) (end 104.775 53.34) (width 1) (layer F.Cu) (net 18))
 (segment (start 79.375 36.195) (end 79.375 37.465) (width 0.5) (layer B.Cu) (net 2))
 (segment (start 71.12 39.37) (end 71.12 40.005) (width 0.5) (layer B.Cu) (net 2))
 (segment (start 72.39 38.1) (end 71.12 39.37) (width 0.5) (layer B.Cu) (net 2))
 (segment (start 78.74 38.1) (end 72.39 38.1) (width 0.5) (layer B.Cu) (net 2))
 (segment (start 79.375 37.465) (end 78.74 38.1) (width 0.5) (layer B.Cu) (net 2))
 (segment (start 72.39 57.785) (end 78.01 57.785) (width 0.5) (layer B.Cu) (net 2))
 (segment (start 71.12 56.515) (end 72.39 57.785) (width 0.5) (layer B.Cu) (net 2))
 (segment (start 71.12 40.005) (end 71.12 56.515) (width 0.5) (layer B.Cu) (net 2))
 (segment (start 78.01 57.785) (end 78.01 61.595) (width 0.5) (layer B.Cu) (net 2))
 (segment (start 77.47 64.675) (end 77.47 62.135) (width 0.5) (layer B.Cu) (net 2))
 (segment (start 77.47 62.135) (end 78.01 61.595) (width 0.5) (layer B.Cu) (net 2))
 (segment (start 73.66 65.175) (end 76.97 65.175) (width 0.5) (layer B.Cu) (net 2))
 (segment (start 76.97 65.175) (end 77.47 64.675) (width 0.5) (layer B.Cu) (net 2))
 (segment (start 118.955 64.135) (end 121.825 64.135) (width 1) (layer F.Cu) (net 10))
 (segment (start 121.825 64.135) (end 123.19 62.77) (width 1) (layer F.Cu) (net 10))
 (segment (start 123.19 62.77) (end 123.19 58.42) (width 1) (layer F.Cu) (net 10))
 (segment (start 123.19 58.42) (end 126.32 58.42) (width 1) (layer F.Cu) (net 10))
 (segment (start 126.32 58.42) (end 128.27 60.37) (width 1) (layer F.Cu) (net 10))
 (segment (start 133.985 60.96) (end 128.86 60.96) (width 1) (layer F.Cu) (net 10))
 (segment (start 128.86 60.96) (end 128.27 60.37) (width 1) (layer F.Cu) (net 10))
 (segment (start 128.27 69.17) (end 128.27 66.04) (width 1) (layer F.Cu) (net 11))
 (segment (start 133.985 66.04) (end 128.27 66.04) (width 1) (layer F.Cu) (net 11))
 (segment (start 128.27 66.04) (end 123.92 66.04) (width 1) (layer F.Cu) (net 11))
 (segment (start 123.92 66.04) (end 123.19 66.77) (width 1) (layer F.Cu) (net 11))
 (segment (start 118.955 66.675) (end 123.095 66.675) (width 1) (layer F.Cu) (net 11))
 (segment (start 123.095 66.675) (end 123.19 66.77) (width 1) (layer F.Cu) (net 11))
 (segment (start 115.57 48.795) (end 115.57 50.8) (width 1) (layer B.Cu) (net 11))
 (segment (start 117.475 66.675) (end 118.955 66.675) (width 1) (layer F.Cu) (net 11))
 (segment (start 116.84 66.04) (end 117.475 66.675) (width 1) (layer F.Cu) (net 11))
 (segment (start 116.84 52.07) (end 116.84 66.04) (width 1) (layer F.Cu) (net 11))
 (segment (start 115.57 50.8) (end 116.84 52.07) (width 1) (layer F.Cu) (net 11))
 (via (at 115.57 50.8) (size 0.6) (drill 0.4) (layers F.Cu B.Cu) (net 11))
 (segment (start 115.57 42.645) (end 115.57 40.64) (width 1) (layer B.Cu) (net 12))
 (segment (start 115.57 40.64) (end 113.03 40.64) (width 1) (layer B.Cu) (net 12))
 (segment (start 113.03 40.64) (end 112.395 41.275) (width 1) (layer B.Cu) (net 12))
 (segment (start 112.395 41.275) (end 112.395 42.545) (width 1) (layer B.Cu) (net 12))
 (segment (start 110.095 37.465) (end 110.095 41.035) (width 1) (layer B.Cu) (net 12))
 (segment (start 110.095 41.035) (end 111.605 42.545) (width 1) (layer B.Cu) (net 12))
 (segment (start 111.605 42.545) (end 112.395 42.545) (width 1) (layer B.Cu) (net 12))
 (segment (start 105.095 37.465) (end 110.095 37.465) (width 1) (layer B.Cu) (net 12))
 (segment (start 112.395 42.545) (end 111.125 42.545) (width 1) (layer F.Cu) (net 12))
 (segment (start 110.095 41.515) (end 110.095 37.465) (width 1) (layer F.Cu) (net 12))
 (segment (start 111.125 42.545) (end 110.095 41.515) (width 1) (layer F.Cu) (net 12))
 (segment (start 105.095 37.465) (end 110.095 37.465) (width 1) (layer F.Cu) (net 12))
 (segment (start 122.395 44.045) (end 122.395 40.64) (width 1) (layer B.Cu) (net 13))
 (segment (start 122.395 40.64) (end 122.555 40.64) (width 1) (layer B.Cu) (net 13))
 (segment (start 118.11 42.645) (end 118.11 40.64) (width 1) (layer B.Cu) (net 13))
 (segment (start 131.445 40.64) (end 132.715 41.91) (width 1) (layer B.Cu) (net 13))
 (segment (start 118.11 40.64) (end 122.555 40.64) (width 1) (layer B.Cu) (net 13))
 (segment (start 122.555 40.64) (end 131.445 40.64) (width 1) (layer B.Cu) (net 13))
 (segment (start 132.715 41.91) (end 133.35 41.91) (width 1) (layer B.Cu) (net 13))
 (segment (start 123.19 48.26) (end 123.19 53.34) (width 1) (layer B.Cu) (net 14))
 (segment (start 127 53.34) (end 133.35 53.34) (width 1) (layer B.Cu) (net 14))
 (segment (start 133.985 63.5) (end 135.89 63.5) (width 1) (layer B.Cu) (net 14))
 (segment (start 135.89 63.5) (end 136.525 62.865) (width 1) (layer B.Cu) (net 14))
 (segment (start 136.525 62.865) (end 136.525 54.61) (width 1) (layer B.Cu) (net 14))
 (segment (start 136.525 54.61) (end 135.255 53.34) (width 1) (layer B.Cu) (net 14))
 (segment (start 135.255 53.34) (end 133.35 53.34) (width 1) (layer B.Cu) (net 14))
 (segment (start 133.985 63.5) (end 135.89 63.5) (width 1) (layer F.Cu) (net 14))
 (segment (start 135.255 53.34) (end 133.35 53.34) (width 1) (layer F.Cu) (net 14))
 (segment (start 136.525 54.61) (end 135.255 53.34) (width 1) (layer F.Cu) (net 14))
 (segment (start 136.525 62.865) (end 136.525 54.61) (width 1) (layer F.Cu) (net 14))
 (segment (start 135.89 63.5) (end 136.525 62.865) (width 1) (layer F.Cu) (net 14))
 (segment (start 123.19 48.26) (end 123.19 53.34) (width 1) (layer F.Cu) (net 14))
 (segment (start 123.19 53.34) (end 127 53.34) (width 1) (layer F.Cu) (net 14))
 (segment (start 127 53.34) (end 133.35 53.34) (width 1) (layer F.Cu) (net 14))
 (segment (start 123.19 53.34) (end 127 53.34) (width 1) (layer B.Cu) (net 14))
 (segment (start 120.095 37.465) (end 125.095 37.465) (width 1) (layer B.Cu) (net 15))
 (segment (start 120.095 37.465) (end 125.095 37.465) (width 1) (layer F.Cu) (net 15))
 (segment (start 125.095 37.465) (end 132.08 37.465) (width 1) (layer F.Cu) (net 15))
 (segment (start 132.08 37.465) (end 132.715 36.83) (width 1) (layer F.Cu) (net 15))
 (segment (start 132.715 36.83) (end 133.35 36.83) (width 1) (layer F.Cu) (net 15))
 (segment (start 125.095 37.465) (end 130.81 37.465) (width 1) (layer B.Cu) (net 15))
 (segment (start 130.81 37.465) (end 132.08 37.465) (width 1) (layer B.Cu) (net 15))
 (segment (start 132.08 37.465) (end 132.715 36.83) (width 1) (layer B.Cu) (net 15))
 (segment (start 132.715 36.83) (end 133.35 36.83) (width 1) (layer B.Cu) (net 15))
 (segment (start 96.52 76.2) (end 96.52 74.93) (width 0.5) (layer B.Cu) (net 7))
 (segment (start 91.44 73.025) (end 91.44 71.755) (width 0.5) (layer B.Cu) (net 7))
 (segment (start 92.71 74.295) (end 91.44 73.025) (width 0.5) (layer B.Cu) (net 7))
 (segment (start 95.885 74.295) (end 92.71 74.295) (width 0.5) (layer B.Cu) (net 7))
 (segment (start 96.52 74.93) (end 95.885 74.295) (width 0.5) (layer B.Cu) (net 7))
 (segment (start 86.36 65.405) (end 86.36 68.58) (width 0.5) (layer B.Cu) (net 16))
 (segment (start 86.36 68.58) (end 86.36 71.755) (width 0.5) (layer B.Cu) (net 16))
 (segment (start 86.36 65.405) (end 83.185 65.405) (width 0.5) (layer B.Cu) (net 16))
 (segment (start 82.01 64.23) (end 82.01 61.595) (width 0.5) (layer B.Cu) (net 16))
 (segment (start 83.185 65.405) (end 82.01 64.23) (width 0.5) (layer B.Cu) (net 16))
 (segment (start 119.38 76.2) (end 119.38 74.93) (width 0.5) (layer B.Cu) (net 6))
 (segment (start 93.98 68.58) (end 91.44 68.58) (width 0.5) (layer B.Cu) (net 6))
 (segment (start 94.615 69.215) (end 93.98 68.58) (width 0.5) (layer B.Cu) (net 6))
 (segment (start 94.615 71.755) (end 94.615 69.215) (width 0.5) (layer B.Cu) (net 6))
 (segment (start 95.885 73.025) (end 94.615 71.755) (width 0.5) (layer B.Cu) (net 6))
 (segment (start 117.475 73.025) (end 95.885 73.025) (width 0.5) (layer B.Cu) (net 6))
 (segment (start 119.38 74.93) (end 117.475 73.025) (width 0.5) (layer B.Cu) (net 6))
 (segment (start 91.44 65.405) (end 94.615 65.405) (width 0.5) (layer B.Cu) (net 5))
 (segment (start 121.92 73.66) (end 121.92 76.2) (width 0.5) (layer B.Cu) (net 5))
 (segment (start 120.015 71.755) (end 121.92 73.66) (width 0.5) (layer B.Cu) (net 5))
 (segment (start 96.52 71.755) (end 120.015 71.755) (width 0.5) (layer B.Cu) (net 5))
 (segment (start 95.885 71.12) (end 96.52 71.755) (width 0.5) (layer B.Cu) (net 5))
 (segment (start 95.885 66.675) (end 95.885 71.12) (width 0.5) (layer B.Cu) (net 5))
 (segment (start 94.615 65.405) (end 95.885 66.675) (width 0.5) (layer B.Cu) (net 5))
 (segment (start 113.455 64.135) (end 111.125 64.135) (width 0.5) (layer F.Cu) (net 17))
 (segment (start 83.82 57.785) (end 82.01 57.785) (width 0.5) (layer B.Cu) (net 17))
 (segment (start 85.09 59.055) (end 83.82 57.785) (width 0.5) (layer B.Cu) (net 17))
 (segment (start 85.09 61.595) (end 85.09 59.055) (width 0.5) (layer B.Cu) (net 17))
 (segment (start 86.36 62.865) (end 85.09 61.595) (width 0.5) (layer B.Cu) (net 17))
 (segment (start 95.885 62.865) (end 86.36 62.865) (width 0.5) (layer B.Cu) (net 17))
 (segment (start 97.155 64.135) (end 95.885 62.865) (width 0.5) (layer B.Cu) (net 17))
 (segment (start 111.125 64.135) (end 97.155 64.135) (width 0.5) (layer B.Cu) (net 17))
 (via (at 111.125 64.135) (size 0.6) (drill 0.4) (layers F.Cu B.Cu) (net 17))
 (segment (start 69.85 64.675) (end 69.85 37.465) (width 0.5) (layer B.Cu) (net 1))
 (segment (start 71.12 36.195) (end 76.835 36.195) (width 0.5) (layer B.Cu) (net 1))
 (segment (start 69.85 37.465) (end 71.12 36.195) (width 0.5) (layer B.Cu) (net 1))
 (segment (start 81.915 41.275) (end 81.915 43.18) (width 0.5) (layer F.Cu) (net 4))
 (segment (start 86.9 44.45) (end 90.805 40.545) (width 0.5) (layer F.Cu) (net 4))
 (segment (start 83.185 44.45) (end 86.9 44.45) (width 0.5) (layer F.Cu) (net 4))
 (segment (start 81.915 43.18) (end 83.185 44.45) (width 0.5) (layer F.Cu) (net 4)))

